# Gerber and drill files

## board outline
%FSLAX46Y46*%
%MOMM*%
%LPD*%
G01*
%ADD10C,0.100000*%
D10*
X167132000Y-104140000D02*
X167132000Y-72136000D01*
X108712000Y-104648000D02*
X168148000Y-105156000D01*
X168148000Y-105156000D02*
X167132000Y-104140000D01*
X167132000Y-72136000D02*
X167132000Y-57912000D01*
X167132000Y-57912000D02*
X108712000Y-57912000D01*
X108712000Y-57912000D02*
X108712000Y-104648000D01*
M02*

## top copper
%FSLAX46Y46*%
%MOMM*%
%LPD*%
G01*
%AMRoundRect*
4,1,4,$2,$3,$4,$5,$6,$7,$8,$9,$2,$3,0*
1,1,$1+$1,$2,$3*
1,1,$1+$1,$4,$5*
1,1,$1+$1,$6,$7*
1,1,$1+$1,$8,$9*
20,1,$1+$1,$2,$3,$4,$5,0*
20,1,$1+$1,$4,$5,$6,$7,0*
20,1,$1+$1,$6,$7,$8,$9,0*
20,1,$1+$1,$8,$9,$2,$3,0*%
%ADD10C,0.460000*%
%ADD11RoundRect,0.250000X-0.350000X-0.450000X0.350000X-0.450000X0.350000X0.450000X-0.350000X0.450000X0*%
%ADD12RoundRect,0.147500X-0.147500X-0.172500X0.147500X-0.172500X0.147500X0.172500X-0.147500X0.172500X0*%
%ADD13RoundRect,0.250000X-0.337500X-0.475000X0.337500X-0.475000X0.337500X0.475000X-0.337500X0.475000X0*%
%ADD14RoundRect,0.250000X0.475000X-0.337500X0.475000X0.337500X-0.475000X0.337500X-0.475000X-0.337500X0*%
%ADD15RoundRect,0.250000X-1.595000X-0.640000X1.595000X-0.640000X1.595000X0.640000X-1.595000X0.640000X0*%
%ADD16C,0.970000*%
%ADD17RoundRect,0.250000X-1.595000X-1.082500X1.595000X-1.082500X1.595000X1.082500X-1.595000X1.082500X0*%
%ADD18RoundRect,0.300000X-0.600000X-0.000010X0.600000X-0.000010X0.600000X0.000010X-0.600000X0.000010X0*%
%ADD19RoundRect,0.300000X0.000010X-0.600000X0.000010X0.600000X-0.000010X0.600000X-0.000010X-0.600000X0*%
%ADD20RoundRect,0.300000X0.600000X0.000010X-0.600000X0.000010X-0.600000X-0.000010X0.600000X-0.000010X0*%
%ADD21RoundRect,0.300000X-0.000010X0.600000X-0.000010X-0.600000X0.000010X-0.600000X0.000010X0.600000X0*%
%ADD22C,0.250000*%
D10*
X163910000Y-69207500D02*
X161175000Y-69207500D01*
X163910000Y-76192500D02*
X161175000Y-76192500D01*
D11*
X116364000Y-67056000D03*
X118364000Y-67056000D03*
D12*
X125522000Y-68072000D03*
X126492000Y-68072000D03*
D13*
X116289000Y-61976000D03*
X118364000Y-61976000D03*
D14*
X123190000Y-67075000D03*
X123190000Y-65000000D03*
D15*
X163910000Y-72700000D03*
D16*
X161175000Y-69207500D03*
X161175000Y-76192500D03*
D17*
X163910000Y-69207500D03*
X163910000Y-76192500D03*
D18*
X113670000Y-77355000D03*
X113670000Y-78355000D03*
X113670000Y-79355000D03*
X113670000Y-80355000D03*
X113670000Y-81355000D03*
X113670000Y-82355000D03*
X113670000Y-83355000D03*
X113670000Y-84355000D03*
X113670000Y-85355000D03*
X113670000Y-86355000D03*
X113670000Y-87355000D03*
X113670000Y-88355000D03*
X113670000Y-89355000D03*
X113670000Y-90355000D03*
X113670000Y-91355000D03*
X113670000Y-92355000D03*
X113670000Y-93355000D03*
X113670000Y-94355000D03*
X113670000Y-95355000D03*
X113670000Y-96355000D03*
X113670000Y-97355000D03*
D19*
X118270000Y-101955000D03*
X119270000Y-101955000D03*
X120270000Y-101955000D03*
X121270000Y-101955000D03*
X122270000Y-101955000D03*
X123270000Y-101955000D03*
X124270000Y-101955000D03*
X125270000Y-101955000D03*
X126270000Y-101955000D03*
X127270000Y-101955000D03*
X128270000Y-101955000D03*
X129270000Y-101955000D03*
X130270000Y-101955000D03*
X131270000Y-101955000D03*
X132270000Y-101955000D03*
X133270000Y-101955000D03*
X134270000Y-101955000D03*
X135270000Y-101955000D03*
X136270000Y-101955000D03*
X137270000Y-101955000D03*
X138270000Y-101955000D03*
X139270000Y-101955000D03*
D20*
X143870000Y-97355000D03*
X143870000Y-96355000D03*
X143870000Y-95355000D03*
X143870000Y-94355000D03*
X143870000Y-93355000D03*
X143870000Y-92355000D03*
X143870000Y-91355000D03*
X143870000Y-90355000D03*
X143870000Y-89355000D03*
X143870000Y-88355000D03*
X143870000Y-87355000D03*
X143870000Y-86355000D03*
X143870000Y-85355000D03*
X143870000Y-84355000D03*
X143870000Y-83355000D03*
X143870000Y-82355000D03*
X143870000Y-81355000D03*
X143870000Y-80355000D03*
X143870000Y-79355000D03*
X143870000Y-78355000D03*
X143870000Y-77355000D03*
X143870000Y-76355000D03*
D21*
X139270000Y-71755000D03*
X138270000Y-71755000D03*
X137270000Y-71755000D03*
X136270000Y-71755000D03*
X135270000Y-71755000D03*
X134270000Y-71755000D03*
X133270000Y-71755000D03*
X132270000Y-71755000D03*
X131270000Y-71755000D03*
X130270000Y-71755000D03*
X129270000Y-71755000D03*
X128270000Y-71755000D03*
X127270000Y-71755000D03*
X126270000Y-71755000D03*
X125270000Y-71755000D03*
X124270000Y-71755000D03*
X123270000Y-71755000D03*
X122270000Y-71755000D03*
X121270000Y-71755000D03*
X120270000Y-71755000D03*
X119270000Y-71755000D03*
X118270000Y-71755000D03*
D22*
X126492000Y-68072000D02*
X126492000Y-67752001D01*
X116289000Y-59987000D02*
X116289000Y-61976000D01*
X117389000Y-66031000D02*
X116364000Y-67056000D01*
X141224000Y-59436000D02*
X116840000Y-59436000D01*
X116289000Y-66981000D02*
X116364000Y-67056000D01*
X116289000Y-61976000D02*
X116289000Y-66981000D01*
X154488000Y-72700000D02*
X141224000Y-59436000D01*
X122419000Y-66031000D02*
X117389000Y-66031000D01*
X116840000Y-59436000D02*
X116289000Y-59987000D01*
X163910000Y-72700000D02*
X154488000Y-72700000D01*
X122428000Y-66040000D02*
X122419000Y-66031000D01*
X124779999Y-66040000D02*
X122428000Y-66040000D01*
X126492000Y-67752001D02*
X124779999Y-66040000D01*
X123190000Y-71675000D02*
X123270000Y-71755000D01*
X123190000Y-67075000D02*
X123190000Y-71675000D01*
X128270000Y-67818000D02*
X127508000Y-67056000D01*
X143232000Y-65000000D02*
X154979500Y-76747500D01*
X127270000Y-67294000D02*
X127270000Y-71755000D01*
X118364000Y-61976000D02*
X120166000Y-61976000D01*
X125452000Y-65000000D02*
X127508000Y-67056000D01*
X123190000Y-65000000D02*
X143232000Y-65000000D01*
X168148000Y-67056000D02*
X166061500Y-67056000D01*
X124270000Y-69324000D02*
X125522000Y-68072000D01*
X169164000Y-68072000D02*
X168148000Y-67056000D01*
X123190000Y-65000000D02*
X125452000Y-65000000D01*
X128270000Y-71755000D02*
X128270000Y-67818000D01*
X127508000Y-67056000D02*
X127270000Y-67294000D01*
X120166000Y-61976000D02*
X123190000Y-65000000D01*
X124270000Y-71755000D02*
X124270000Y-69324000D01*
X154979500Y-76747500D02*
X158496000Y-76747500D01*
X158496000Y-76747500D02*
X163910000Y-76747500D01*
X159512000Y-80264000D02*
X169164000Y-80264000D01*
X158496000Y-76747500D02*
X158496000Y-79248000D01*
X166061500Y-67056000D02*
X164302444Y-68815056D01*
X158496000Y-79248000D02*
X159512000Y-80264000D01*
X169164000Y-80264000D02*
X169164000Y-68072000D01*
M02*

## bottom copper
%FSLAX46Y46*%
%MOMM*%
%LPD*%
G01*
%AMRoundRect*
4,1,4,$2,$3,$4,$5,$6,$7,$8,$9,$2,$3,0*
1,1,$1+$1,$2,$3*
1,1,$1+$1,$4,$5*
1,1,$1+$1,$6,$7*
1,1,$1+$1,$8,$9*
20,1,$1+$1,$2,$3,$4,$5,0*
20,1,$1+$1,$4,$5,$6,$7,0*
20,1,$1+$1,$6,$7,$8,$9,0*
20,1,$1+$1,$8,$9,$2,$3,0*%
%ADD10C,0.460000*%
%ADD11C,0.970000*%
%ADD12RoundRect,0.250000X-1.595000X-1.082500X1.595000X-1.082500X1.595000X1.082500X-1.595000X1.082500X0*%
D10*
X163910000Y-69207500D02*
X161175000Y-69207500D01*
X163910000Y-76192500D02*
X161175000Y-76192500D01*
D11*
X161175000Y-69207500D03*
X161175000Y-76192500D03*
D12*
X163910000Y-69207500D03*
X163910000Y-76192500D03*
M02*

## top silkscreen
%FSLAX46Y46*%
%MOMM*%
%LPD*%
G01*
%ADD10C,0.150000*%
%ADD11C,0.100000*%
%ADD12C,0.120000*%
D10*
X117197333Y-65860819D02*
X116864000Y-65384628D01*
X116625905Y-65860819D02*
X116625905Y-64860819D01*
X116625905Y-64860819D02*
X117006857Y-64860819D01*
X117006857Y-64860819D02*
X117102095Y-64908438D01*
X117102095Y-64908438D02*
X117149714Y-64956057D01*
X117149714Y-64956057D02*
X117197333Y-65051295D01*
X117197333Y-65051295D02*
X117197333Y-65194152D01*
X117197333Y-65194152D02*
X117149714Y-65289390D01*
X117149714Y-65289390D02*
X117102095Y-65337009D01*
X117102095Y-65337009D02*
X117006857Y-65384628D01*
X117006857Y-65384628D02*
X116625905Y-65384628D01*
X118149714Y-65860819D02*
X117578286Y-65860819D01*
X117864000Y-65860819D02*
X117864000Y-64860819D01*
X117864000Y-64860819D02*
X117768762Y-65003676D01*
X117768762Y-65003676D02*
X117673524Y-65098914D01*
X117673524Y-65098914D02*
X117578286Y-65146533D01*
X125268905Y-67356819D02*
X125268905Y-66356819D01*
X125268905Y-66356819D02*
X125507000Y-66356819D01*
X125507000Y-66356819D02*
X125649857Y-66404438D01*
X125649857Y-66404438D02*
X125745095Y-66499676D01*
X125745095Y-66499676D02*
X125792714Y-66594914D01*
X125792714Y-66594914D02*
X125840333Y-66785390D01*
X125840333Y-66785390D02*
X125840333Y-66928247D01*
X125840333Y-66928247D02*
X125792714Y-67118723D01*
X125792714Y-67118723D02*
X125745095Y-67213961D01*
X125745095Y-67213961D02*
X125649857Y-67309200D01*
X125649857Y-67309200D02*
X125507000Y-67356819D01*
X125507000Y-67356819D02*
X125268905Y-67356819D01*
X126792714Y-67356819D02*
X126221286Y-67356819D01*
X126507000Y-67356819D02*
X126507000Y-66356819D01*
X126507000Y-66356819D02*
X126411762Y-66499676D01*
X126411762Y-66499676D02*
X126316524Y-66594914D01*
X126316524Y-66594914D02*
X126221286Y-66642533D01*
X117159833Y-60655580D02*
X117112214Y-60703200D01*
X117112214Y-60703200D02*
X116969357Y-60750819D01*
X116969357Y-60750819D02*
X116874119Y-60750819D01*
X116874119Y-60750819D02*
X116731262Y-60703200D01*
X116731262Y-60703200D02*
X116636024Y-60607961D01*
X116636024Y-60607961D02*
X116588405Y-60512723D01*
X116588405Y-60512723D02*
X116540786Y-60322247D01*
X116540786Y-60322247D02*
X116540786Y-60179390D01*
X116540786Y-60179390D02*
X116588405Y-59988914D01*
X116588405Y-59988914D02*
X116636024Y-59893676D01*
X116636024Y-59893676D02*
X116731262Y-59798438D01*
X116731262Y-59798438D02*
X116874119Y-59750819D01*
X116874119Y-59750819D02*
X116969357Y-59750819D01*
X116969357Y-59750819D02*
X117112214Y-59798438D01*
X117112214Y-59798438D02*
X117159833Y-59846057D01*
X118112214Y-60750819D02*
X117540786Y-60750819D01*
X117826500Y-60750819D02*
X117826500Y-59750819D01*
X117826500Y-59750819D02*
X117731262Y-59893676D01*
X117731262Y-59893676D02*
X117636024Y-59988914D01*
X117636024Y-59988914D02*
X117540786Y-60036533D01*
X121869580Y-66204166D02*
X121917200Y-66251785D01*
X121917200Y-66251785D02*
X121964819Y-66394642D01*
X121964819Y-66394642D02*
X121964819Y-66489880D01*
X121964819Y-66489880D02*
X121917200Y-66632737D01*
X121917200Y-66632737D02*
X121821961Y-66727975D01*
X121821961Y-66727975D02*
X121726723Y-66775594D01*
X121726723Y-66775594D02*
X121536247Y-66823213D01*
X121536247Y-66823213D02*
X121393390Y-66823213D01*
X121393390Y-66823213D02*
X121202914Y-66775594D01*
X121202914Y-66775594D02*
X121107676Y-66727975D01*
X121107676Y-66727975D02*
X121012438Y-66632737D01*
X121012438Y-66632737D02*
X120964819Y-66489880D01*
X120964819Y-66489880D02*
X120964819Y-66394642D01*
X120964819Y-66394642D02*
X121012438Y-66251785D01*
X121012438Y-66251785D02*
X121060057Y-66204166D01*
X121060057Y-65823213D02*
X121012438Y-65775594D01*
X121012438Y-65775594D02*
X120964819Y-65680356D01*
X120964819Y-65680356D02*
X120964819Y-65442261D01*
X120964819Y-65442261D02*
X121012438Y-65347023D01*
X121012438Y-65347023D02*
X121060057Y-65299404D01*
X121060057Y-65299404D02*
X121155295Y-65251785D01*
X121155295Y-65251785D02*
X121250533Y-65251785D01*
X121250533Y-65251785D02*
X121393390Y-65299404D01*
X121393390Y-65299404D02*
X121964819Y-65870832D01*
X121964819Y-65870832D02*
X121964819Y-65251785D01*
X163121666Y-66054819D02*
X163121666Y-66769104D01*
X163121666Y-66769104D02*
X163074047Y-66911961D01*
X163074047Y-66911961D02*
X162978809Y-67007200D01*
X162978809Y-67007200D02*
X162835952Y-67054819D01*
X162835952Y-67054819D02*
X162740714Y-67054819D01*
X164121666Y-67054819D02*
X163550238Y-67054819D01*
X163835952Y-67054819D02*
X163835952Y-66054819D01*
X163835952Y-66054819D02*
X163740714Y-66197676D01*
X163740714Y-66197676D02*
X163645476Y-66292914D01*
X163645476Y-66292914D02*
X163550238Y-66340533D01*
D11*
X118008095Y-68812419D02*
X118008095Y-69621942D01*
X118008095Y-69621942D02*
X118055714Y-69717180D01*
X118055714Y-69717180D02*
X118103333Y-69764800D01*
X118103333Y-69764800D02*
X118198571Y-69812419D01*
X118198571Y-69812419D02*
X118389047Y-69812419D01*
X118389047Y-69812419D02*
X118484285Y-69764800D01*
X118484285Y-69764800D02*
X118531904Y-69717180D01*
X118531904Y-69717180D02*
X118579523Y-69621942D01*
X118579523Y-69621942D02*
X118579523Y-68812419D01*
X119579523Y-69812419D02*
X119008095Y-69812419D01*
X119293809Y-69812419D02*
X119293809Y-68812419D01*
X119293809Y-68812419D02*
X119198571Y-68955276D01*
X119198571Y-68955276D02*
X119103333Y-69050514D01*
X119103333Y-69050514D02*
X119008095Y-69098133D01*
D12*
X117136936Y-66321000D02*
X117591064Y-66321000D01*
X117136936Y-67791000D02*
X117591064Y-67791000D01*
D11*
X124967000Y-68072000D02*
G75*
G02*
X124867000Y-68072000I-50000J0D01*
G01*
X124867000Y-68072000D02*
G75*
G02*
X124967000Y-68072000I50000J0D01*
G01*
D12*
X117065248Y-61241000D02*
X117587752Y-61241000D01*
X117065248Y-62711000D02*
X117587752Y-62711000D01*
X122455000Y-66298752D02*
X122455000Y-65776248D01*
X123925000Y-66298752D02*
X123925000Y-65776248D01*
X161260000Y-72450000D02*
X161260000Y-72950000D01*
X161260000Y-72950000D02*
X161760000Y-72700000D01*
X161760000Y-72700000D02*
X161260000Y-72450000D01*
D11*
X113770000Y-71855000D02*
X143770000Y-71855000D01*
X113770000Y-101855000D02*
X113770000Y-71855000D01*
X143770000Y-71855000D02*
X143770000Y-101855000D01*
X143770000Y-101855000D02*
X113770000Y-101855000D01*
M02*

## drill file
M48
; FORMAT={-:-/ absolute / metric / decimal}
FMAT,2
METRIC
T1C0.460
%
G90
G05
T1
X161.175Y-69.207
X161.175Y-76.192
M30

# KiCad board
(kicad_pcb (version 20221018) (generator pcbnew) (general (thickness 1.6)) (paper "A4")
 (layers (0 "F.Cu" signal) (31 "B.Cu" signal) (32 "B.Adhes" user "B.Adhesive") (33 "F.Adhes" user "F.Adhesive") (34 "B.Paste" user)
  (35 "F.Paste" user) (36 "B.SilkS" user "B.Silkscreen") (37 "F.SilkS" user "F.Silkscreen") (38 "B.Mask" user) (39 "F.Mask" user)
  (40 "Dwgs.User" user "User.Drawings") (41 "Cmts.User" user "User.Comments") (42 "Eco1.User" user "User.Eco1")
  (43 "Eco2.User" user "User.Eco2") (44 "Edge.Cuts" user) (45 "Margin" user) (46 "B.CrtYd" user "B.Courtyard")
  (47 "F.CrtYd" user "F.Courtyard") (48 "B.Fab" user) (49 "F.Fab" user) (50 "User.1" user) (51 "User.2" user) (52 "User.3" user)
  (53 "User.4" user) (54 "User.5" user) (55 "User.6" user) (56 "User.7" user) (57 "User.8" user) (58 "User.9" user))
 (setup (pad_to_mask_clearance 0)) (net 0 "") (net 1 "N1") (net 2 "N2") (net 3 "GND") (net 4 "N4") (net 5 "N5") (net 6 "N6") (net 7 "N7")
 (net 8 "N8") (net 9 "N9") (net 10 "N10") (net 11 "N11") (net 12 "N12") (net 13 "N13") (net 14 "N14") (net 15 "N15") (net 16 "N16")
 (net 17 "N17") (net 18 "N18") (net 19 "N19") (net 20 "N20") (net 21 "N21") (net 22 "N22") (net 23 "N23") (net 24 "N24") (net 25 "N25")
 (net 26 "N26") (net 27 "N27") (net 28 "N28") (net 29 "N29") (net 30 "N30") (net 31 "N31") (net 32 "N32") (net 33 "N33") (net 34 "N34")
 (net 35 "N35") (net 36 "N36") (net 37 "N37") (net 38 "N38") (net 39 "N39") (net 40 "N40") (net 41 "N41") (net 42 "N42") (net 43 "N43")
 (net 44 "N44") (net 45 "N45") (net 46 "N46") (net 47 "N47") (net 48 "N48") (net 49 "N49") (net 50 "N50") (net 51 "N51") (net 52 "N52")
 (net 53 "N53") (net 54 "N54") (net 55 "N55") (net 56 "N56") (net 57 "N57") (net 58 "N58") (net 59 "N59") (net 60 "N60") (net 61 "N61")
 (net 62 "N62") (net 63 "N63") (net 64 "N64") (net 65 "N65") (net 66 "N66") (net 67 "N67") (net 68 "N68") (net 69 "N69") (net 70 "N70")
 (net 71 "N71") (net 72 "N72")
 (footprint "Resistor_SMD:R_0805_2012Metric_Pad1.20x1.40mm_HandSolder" (layer "F.Cu") (at 117.364 67.056)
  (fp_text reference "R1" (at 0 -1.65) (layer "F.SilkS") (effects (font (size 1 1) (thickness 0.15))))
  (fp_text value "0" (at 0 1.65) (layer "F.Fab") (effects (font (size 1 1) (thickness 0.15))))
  (fp_line (start -0.227064 -0.735) (end 0.227064 -0.735) (stroke (width 0.12) (type solid)) (layer "F.SilkS"))
  (fp_line (start -0.227064 0.735) (end 0.227064 0.735) (stroke (width 0.12) (type solid)) (layer "F.SilkS"))
  (pad "1" smd roundrect (at -1 0) (size 1.2 1.4) (layers "F.Cu" "F.Paste" "F.Mask") (roundrect_rratio 0.208333) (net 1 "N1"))
  (pad "2" smd roundrect (at 1 0) (size 1.2 1.4) (layers "F.Cu" "F.Paste" "F.Mask") (roundrect_rratio 0.208333) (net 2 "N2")))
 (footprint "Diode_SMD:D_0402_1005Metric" (layer "F.Cu") (at 126.007 68.072)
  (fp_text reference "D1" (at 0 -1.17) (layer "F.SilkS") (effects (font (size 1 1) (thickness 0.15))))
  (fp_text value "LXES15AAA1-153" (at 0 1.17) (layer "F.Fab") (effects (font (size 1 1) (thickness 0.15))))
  (fp_circle (center -1.09 0) (end -1.04 0) (stroke (width 0.1) (type solid)) (fill none) (layer "F.SilkS"))
  (pad "1" smd roundrect (at -0.485 0) (size 0.59 0.64) (layers "F.Cu" "F.Paste" "F.Mask") (roundrect_rratio 0.25) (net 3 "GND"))
  (pad "2" smd roundrect (at 0.485 0) (size 0.59 0.64) (layers "F.Cu" "F.Paste" "F.Mask") (roundrect_rratio 0.25) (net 1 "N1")))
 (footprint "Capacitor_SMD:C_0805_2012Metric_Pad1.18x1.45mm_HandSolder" (layer "F.Cu") (at 117.3265 61.976)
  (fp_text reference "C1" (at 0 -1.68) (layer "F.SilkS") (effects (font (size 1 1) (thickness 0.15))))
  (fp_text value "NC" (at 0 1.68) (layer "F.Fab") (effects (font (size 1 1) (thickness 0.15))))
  (fp_line (start -0.261252 -0.735) (end 0.261252 -0.735) (stroke (width 0.12) (type solid)) (layer "F.SilkS"))
  (fp_line (start -0.261252 0.735) (end 0.261252 0.735) (stroke (width 0.12) (type solid)) (layer "F.SilkS"))
  (pad "1" smd roundrect (at -1.0375 0) (size 1.175 1.45) (layers "F.Cu" "F.Paste" "F.Mask") (roundrect_rratio 0.212766) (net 1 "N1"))
  (pad "2" smd roundrect (at 1.0375 0) (size 1.175 1.45) (layers "F.Cu" "F.Paste" "F.Mask") (roundrect_rratio 0.212766) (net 3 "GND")))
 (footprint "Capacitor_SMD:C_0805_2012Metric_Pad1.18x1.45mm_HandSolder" (layer "F.Cu") (at 123.19 66.0375 90)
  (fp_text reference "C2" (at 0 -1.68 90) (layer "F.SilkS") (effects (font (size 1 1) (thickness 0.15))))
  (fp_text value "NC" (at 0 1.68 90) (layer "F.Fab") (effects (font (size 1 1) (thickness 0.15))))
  (fp_line (start -0.261252 -0.735) (end 0.261252 -0.735) (stroke (width 0.12) (type solid)) (layer "F.SilkS"))
  (fp_line (start -0.261252 0.735) (end 0.261252 0.735) (stroke (width 0.12) (type solid)) (layer "F.SilkS"))
  (pad "1" smd roundrect (at -1.0375 0 90) (size 1.175 1.45) (layers "F.Cu" "F.Paste" "F.Mask") (roundrect_rratio 0.212766) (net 2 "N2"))
  (pad "2" smd roundrect (at 1.0375 0 90) (size 1.175 1.45) (layers "F.Cu" "F.Paste" "F.Mask") (roundrect_rratio 0.212766) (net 3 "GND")))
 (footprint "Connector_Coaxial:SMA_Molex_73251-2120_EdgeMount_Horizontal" (layer "F.Cu") (at 164.16 72.7)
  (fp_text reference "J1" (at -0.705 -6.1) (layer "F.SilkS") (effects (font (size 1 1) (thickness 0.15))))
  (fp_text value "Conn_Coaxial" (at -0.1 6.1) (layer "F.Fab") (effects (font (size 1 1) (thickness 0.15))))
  (fp_line (start -0.25 -3.4925) (end -2.985 -3.4925) (stroke (width 0.46) (type default)) (layer "F.Cu"))
  (fp_line (start -0.25 3.4925) (end -2.985 3.4925) (stroke (width 0.46) (type default)) (layer "F.Cu"))
  (fp_line (start -0.25 -3.4925) (end -2.985 -3.4925) (stroke (width 0.46) (type default)) (layer "B.Cu"))
  (fp_line (start -0.25 3.4925) (end -2.985 3.4925) (stroke (width 0.46) (type default)) (layer "B.Cu"))
  (fp_line (start -2.9 -0.25) (end -2.9 0.25) (stroke (width 0.12) (type solid)) (layer "F.SilkS"))
  (fp_line (start -2.9 0.25) (end -2.4 0) (stroke (width 0.12) (type solid)) (layer "F.SilkS"))
  (fp_line (start -2.4 0) (end -2.9 -0.25) (stroke (width 0.12) (type solid)) (layer "F.SilkS"))
  (pad "1" smd roundrect (at -0.25 0) (size 3.69 1.78) (layers "F.Cu" "F.Paste" "F.Mask") (roundrect_rratio 0.1404494382) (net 1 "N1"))
  (pad "2" thru_hole circle (at -2.985 -3.4925) (size 0.97 0.97) (drill 0.46) (layers "*.Cu") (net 3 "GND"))
  (pad "2" thru_hole circle (at -2.985 3.4925) (size 0.97 0.97) (drill 0.46) (layers "*.Cu") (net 3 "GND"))
  (pad "2" smd roundrect (at -0.25 -3.4925) (size 3.69 2.665) (layers "F.Cu" "F.Paste" "F.Mask") (roundrect_rratio 0.09380863039)
   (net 3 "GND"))
  (pad "2" smd roundrect (at -0.25 -3.4925) (size 3.69 2.665) (layers "B.Cu" "B.Paste" "B.Mask") (roundrect_rratio 0.09380863039)
   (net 3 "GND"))
  (pad "2" smd roundrect (at -0.25 3.4925) (size 3.69 2.665) (layers "F.Cu" "F.Paste" "F.Mask") (roundrect_rratio 0.09380863039)
   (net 3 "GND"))
  (pad "2" smd roundrect (at -0.25 3.4925) (size 3.69 2.665) (layers "B.Cu" "B.Paste" "B.Mask") (roundrect_rratio 0.09380863039)
   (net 3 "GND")))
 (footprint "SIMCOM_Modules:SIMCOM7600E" (layer "F.Cu") (at 128.77 86.855)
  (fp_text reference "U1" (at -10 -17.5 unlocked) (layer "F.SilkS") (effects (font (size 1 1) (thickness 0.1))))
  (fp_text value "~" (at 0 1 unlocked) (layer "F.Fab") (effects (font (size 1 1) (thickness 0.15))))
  (fp_line (start -15 -15) (end 15 -15) (stroke (width 0.1) (type default)) (layer "F.SilkS"))
  (fp_line (start -15 15) (end -15 -15) (stroke (width 0.1) (type default)) (layer "F.SilkS"))
  (fp_line (start 15 -15) (end 15 15) (stroke (width 0.1) (type default)) (layer "F.SilkS"))
  (fp_line (start 15 15) (end -15 15) (stroke (width 0.1) (type default)) (layer "F.SilkS"))
  (pad "1" smd roundrect (at -15.1 -9.5) (size 1.8 0.6) (layers "F.Cu" "F.Paste" "F.Mask") (roundrect_rratio 0.5) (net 3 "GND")
   (thermal_bridge_angle 45))
  (pad "2" smd roundrect (at -15.1 -8.5) (size 1.8 0.6) (layers "F.Cu" "F.Paste" "F.Mask") (roundrect_rratio 0.5) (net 3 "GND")
   (thermal_bridge_angle 45))
  (pad "3" smd roundrect (at -15.1 -7.5) (size 1.8 0.6) (layers "F.Cu" "F.Paste" "F.Mask") (roundrect_rratio 0.5) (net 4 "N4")
   (thermal_bridge_angle 45))
  (pad "4" smd roundrect (at -15.1 -6.5) (size 1.8 0.6) (layers "F.Cu" "F.Paste" "F.Mask") (roundrect_rratio 0.5) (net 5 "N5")
   (thermal_bridge_angle 45))
  (pad "5" smd roundrect (at -15.1 -5.5) (size 1.8 0.6) (layers "F.Cu" "F.Paste" "F.Mask") (roundrect_rratio 0.5) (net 3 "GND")
   (thermal_bridge_angle 45))
  (pad "6" smd roundrect (at -15.1 -4.5) (size 1.8 0.6) (layers "F.Cu" "F.Paste" "F.Mask") (roundrect_rratio 0.5) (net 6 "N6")
   (thermal_bridge_angle 45))
  (pad "7" smd roundrect (at -15.1 -3.5) (size 1.8 0.6) (layers "F.Cu" "F.Paste" "F.Mask") (roundrect_rratio 0.5) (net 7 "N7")
   (thermal_bridge_angle 45))
  (pad "8" smd roundrect (at -15.1 -2.5) (size 1.8 0.6) (layers "F.Cu" "F.Paste" "F.Mask") (roundrect_rratio 0.5) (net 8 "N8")
   (thermal_bridge_angle 45))
  (pad "9" smd roundrect (at -15.1 -1.5) (size 1.8 0.6) (layers "F.Cu" "F.Paste" "F.Mask") (roundrect_rratio 0.5) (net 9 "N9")
   (thermal_bridge_angle 45))
  (pad "10" smd roundrect (at -15.1 -0.5) (size 1.8 0.6) (layers "F.Cu" "F.Paste" "F.Mask") (roundrect_rratio 0.5) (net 3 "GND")
   (thermal_bridge_angle 45))
  (pad "11" smd roundrect (at -15.1 0.5) (size 1.8 0.6) (layers "F.Cu" "F.Paste" "F.Mask") (roundrect_rratio 0.5) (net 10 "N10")
   (thermal_bridge_angle 45))
  (pad "12" smd roundrect (at -15.1 1.5) (size 1.8 0.6) (layers "F.Cu" "F.Paste" "F.Mask") (roundrect_rratio 0.5) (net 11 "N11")
   (thermal_bridge_angle 45))
  (pad "13" smd roundrect (at -15.1 2.5) (size 1.8 0.6) (layers "F.Cu" "F.Paste" "F.Mask") (roundrect_rratio 0.5) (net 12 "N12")
   (thermal_bridge_angle 45))
  (pad "14" smd roundrect (at -15.1 3.5) (size 1.8 0.6) (layers "F.Cu" "F.Paste" "F.Mask") (roundrect_rratio 0.5) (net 3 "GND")
   (thermal_bridge_angle 45))
  (pad "15" smd roundrect (at -15.1 4.5) (size 1.8 0.6) (layers "F.Cu" "F.Paste" "F.Mask") (roundrect_rratio 0.5) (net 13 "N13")
   (thermal_bridge_angle 45))
  (pad "16" smd roundrect (at -15.1 5.5) (size 1.8 0.6) (layers "F.Cu" "F.Paste" "F.Mask") (roundrect_rratio 0.5) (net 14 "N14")
   (thermal_bridge_angle 45))
  (pad "17" smd roundrect (at -15.1 6.5) (size 1.8 0.6) (layers "F.Cu" "F.Paste" "F.Mask") (roundrect_rratio 0.5) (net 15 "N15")
   (thermal_bridge_angle 45))
  (pad "18" smd roundrect (at -15.1 7.5) (size 1.8 0.6) (layers "F.Cu" "F.Paste" "F.Mask") (roundrect_rratio 0.5) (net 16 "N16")
   (thermal_bridge_angle 45))
  (pad "19" smd roundrect (at -15.1 8.5) (size 1.8 0.6) (layers "F.Cu" "F.Paste" "F.Mask") (roundrect_rratio 0.5) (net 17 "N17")
   (thermal_bridge_angle 45))
  (pad "20" smd roundrect (at -15.1 9.5) (size 1.8 0.6) (layers "F.Cu" "F.Paste" "F.Mask") (roundrect_rratio 0.5) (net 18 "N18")
   (thermal_bridge_angle 45))
  (pad "21" smd roundrect (at -15.1 10.5) (size 1.8 0.6) (layers "F.Cu" "F.Paste" "F.Mask") (roundrect_rratio 0.5) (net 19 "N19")
   (thermal_bridge_angle 45))
  (pad "22" smd roundrect (at -10.5 15.1 90) (size 1.8 0.6) (layers "F.Cu" "F.Paste" "F.Mask") (roundrect_rratio 0.5) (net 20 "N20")
   (thermal_bridge_angle 45))
  (pad "23" smd roundrect (at -9.5 15.1 90) (size 1.8 0.6) (layers "F.Cu" "F.Paste" "F.Mask") (roundrect_rratio 0.5) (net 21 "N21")
   (thermal_bridge_angle 45))
  (pad "24" smd roundrect (at -8.5 15.1 90) (size 1.8 0.6) (layers "F.Cu" "F.Paste" "F.Mask") (roundrect_rratio 0.5) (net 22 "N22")
   (thermal_bridge_angle 45))
  (pad "25" smd roundrect (at -7.5 15.1 90) (size 1.8 0.6) (layers "F.Cu" "F.Paste" "F.Mask") (roundrect_rratio 0.5) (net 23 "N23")
   (thermal_bridge_angle 45))
  (pad "26" smd roundrect (at -6.5 15.1 90) (size 1.8 0.6) (layers "F.Cu" "F.Paste" "F.Mask") (roundrect_rratio 0.5) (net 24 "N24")
   (thermal_bridge_angle 45))
  (pad "27" smd roundrect (at -5.5 15.1 90) (size 1.8 0.6) (layers "F.Cu" "F.Paste" "F.Mask") (roundrect_rratio 0.5) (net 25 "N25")
   (thermal_bridge_angle 45))
  (pad "28" smd roundrect (at -4.5 15.1 90) (size 1.8 0.6) (layers "F.Cu" "F.Paste" "F.Mask") (roundrect_rratio 0.5) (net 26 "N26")
   (thermal_bridge_angle 45))
  (pad "29" smd roundrect (at -3.5 15.1 90) (size 1.8 0.6) (layers "F.Cu" "F.Paste" "F.Mask") (roundrect_rratio 0.5) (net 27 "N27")
   (thermal_bridge_angle 45))
  (pad "30" smd roundrect (at -2.5 15.1 90) (size 1.8 0.6) (layers "F.Cu" "F.Paste" "F.Mask") (roundrect_rratio 0.5) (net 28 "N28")
   (thermal_bridge_angle 45))
  (pad "31" smd roundrect (at -1.5 15.1 90) (size 1.8 0.6) (layers "F.Cu" "F.Paste" "F.Mask") (roundrect_rratio 0.5) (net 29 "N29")
   (thermal_bridge_angle 45))
  (pad "32" smd roundrect (at -0.5 15.1 90) (size 1.8 0.6) (layers "F.Cu" "F.Paste" "F.Mask") (roundrect_rratio 0.5) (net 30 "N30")
   (thermal_bridge_angle 45))
  (pad "33" smd roundrect (at 0.5 15.1 90) (size 1.8 0.6) (layers "F.Cu" "F.Paste" "F.Mask") (roundrect_rratio 0.5) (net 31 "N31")
   (thermal_bridge_angle 45))
  (pad "34" smd roundrect (at 1.5 15.1 90) (size 1.8 0.6) (layers "F.Cu" "F.Paste" "F.Mask") (roundrect_rratio 0.5) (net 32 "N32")
   (thermal_bridge_angle 45))
  (pad "35" smd roundrect (at 2.5 15.1 90) (size 1.8 0.6) (layers "F.Cu" "F.Paste" "F.Mask") (roundrect_rratio 0.5) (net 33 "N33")
   (thermal_bridge_angle 45))
  (pad "36" smd roundrect (at 3.5 15.1 90) (size 1.8 0.6) (layers "F.Cu" "F.Paste" "F.Mask") (roundrect_rratio 0.5) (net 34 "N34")
   (thermal_bridge_angle 45))
  (pad "37" smd roundrect (at 4.5 15.1 90) (size 1.8 0.6) (layers "F.Cu" "F.Paste" "F.Mask") (roundrect_rratio 0.5) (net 3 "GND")
   (thermal_bridge_angle 45))
  (pad "38" smd roundrect (at 5.5 15.1 90) (size 1.8 0.6) (layers "F.Cu" "F.Paste" "F.Mask") (roundrect_rratio 0.5) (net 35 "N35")
   (thermal_bridge_angle 45))
  (pad "39" smd roundrect (at 6.5 15.1 90) (size 1.8 0.6) (layers "F.Cu" "F.Paste" "F.Mask") (roundrect_rratio 0.5) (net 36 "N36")
   (thermal_bridge_angle 45))
  (pad "40" smd roundrect (at 7.5 15.1 90) (size 1.8 0.6) (layers "F.Cu" "F.Paste" "F.Mask") (roundrect_rratio 0.5) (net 3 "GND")
   (thermal_bridge_angle 45))
  (pad "41" smd roundrect (at 8.5 15.1 90) (size 1.8 0.6) (layers "F.Cu" "F.Paste" "F.Mask") (roundrect_rratio 0.5) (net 3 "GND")
   (thermal_bridge_angle 45))
  (pad "42" smd roundrect (at 9.5 15.1 90) (size 1.8 0.6) (layers "F.Cu" "F.Paste" "F.Mask") (roundrect_rratio 0.5) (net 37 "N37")
   (thermal_bridge_angle 45))
  (pad "43" smd roundrect (at 10.5 15.1 90) (size 1.8 0.6) (layers "F.Cu" "F.Paste" "F.Mask") (roundrect_rratio 0.5) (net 3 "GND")
   (thermal_bridge_angle 45))
  (pad "44" smd roundrect (at 15.1 10.5 180) (size 1.8 0.6) (layers "F.Cu" "F.Paste" "F.Mask") (roundrect_rratio 0.5) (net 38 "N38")
   (thermal_bridge_angle 45))
  (pad "45" smd roundrect (at 15.1 9.5 180) (size 1.8 0.6) (layers "F.Cu" "F.Paste" "F.Mask") (roundrect_rratio 0.5) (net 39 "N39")
   (thermal_bridge_angle 45))
  (pad "46" smd roundrect (at 15.1 8.5 180) (size 1.8 0.6) (layers "F.Cu" "F.Paste" "F.Mask") (roundrect_rratio 0.5) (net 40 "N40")
   (thermal_bridge_angle 45))
  (pad "47" smd roundrect (at 15.1 7.5 180) (size 1.8 0.6) (layers "F.Cu" "F.Paste" "F.Mask") (roundrect_rratio 0.5) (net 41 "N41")
   (thermal_bridge_angle 45))
  (pad "48" smd roundrect (at 15.1 6.5 180) (size 1.8 0.6) (layers "F.Cu" "F.Paste" "F.Mask") (roundrect_rratio 0.5) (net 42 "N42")
   (thermal_bridge_angle 45))
  (pad "49" smd roundrect (at 15.1 5.5 180) (size 1.8 0.6) (layers "F.Cu" "F.Paste" "F.Mask") (roundrect_rratio 0.5) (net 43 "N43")
   (thermal_bridge_angle 45))
  (pad "50" smd roundrect (at 15.1 4.5 180) (size 1.8 0.6) (layers "F.Cu" "F.Paste" "F.Mask") (roundrect_rratio 0.5) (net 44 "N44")
   (thermal_bridge_angle 45))
  (pad "51" smd roundrect (at 15.1 3.5 180) (size 1.8 0.6) (layers "F.Cu" "F.Paste" "F.Mask") (roundrect_rratio 0.5) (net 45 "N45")
   (thermal_bridge_angle 45))
  (pad "52" smd roundrect (at 15.1 2.5 180) (size 1.8 0.6) (layers "F.Cu" "F.Paste" "F.Mask") (roundrect_rratio 0.5) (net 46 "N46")
   (thermal_bridge_angle 45))
  (pad "53" smd roundrect (at 15.1 1.5 180) (size 1.8 0.6) (layers "F.Cu" "F.Paste" "F.Mask") (roundrect_rratio 0.5) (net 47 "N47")
   (thermal_bridge_angle 45))
  (pad "54" smd roundrect (at 15.1 0.5 180) (size 1.8 0.6) (layers "F.Cu" "F.Paste" "F.Mask") (roundrect_rratio 0.5) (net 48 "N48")
   (thermal_bridge_angle 45))
  (pad "55" smd roundrect (at 15.1 -0.5 180) (size 1.8 0.6) (layers "F.Cu" "F.Paste" "F.Mask") (roundrect_rratio 0.5) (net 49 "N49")
   (thermal_bridge_angle 45))
  (pad "56" smd roundrect (at 15.1 -1.5 180) (size 1.8 0.6) (layers "F.Cu" "F.Paste" "F.Mask") (roundrect_rratio 0.5) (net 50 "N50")
   (thermal_bridge_angle 45))
  (pad "57" smd roundrect (at 15.1 -2.5 180) (size 1.8 0.6) (layers "F.Cu" "F.Paste" "F.Mask") (roundrect_rratio 0.5) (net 3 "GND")
   (thermal_bridge_angle 45))
  (pad "58" smd roundrect (at 15.1 -3.5 180) (size 1.8 0.6) (layers "F.Cu" "F.Paste" "F.Mask") (roundrect_rratio 0.5) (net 3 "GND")
   (thermal_bridge_angle 45))
  (pad "59" smd roundrect (at 15.1 -4.5 180) (size 1.8 0.6) (layers "F.Cu" "F.Paste" "F.Mask") (roundrect_rratio 0.5) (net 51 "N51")
   (thermal_bridge_angle 45))
  (pad "60" smd roundrect (at 15.1 -5.5 180) (size 1.8 0.6) (layers "F.Cu" "F.Paste" "F.Mask") (roundrect_rratio 0.5) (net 3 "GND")
   (thermal_bridge_angle 45))
  (pad "61" smd roundrect (at 15.1 -6.5 180) (size 1.8 0.6) (layers "F.Cu" "F.Paste" "F.Mask") (roundrect_rratio 0.5) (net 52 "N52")
   (thermal_bridge_angle 45))
  (pad "62" smd roundrect (at 15.1 -7.5 180) (size 1.8 0.6) (layers "F.Cu" "F.Paste" "F.Mask") (roundrect_rratio 0.5) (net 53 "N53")
   (thermal_bridge_angle 45))
  (pad "63" smd roundrect (at 15.1 -8.5 180) (size 1.8 0.6) (layers "F.Cu" "F.Paste" "F.Mask") (roundrect_rratio 0.5) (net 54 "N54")
   (thermal_bridge_angle 45))
  (pad "64" smd roundrect (at 15.1 -9.5 180) (size 1.8 0.6) (layers "F.Cu" "F.Paste" "F.Mask") (roundrect_rratio 0.5) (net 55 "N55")
   (thermal_bridge_angle 45))
  (pad "65" smd roundrect (at 15.1 -10.5 180) (size 1.8 0.6) (layers "F.Cu" "F.Paste" "F.Mask") (roundrect_rratio 0.5) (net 3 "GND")
   (thermal_bridge_angle 45))
  (pad "66" smd roundrect (at 10.5 -15.1 270) (size 1.8 0.6) (layers "F.Cu" "F.Paste" "F.Mask") (roundrect_rratio 0.5) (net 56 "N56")
   (thermal_bridge_angle 45))
  (pad "67" smd roundrect (at 9.5 -15.1 270) (size 1.8 0.6) (layers "F.Cu" "F.Paste" "F.Mask") (roundrect_rratio 0.5) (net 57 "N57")
   (thermal_bridge_angle 45))
  (pad "68" smd roundrect (at 8.5 -15.1 270) (size 1.8 0.6) (layers "F.Cu" "F.Paste" "F.Mask") (roundrect_rratio 0.5) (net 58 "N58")
   (thermal_bridge_angle 45))
  (pad "69" smd roundrect (at 7.5 -15.1 270) (size 1.8 0.6) (layers "F.Cu" "F.Paste" "F.Mask") (roundrect_rratio 0.5) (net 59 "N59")
   (thermal_bridge_angle 45))
  (pad "70" smd roundrect (at 6.5 -15.1 270) (size 1.8 0.6) (layers "F.Cu" "F.Paste" "F.Mask") (roundrect_rratio 0.5) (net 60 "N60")
   (thermal_bridge_angle 45))
  (pad "71" smd roundrect (at 5.5 -15.1 270) (size 1.8 0.6) (layers "F.Cu" "F.Paste" "F.Mask") (roundrect_rratio 0.5) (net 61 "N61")
   (thermal_bridge_angle 45))
  (pad "72" smd roundrect (at 4.5 -15.1 270) (size 1.8 0.6) (layers "F.Cu" "F.Paste" "F.Mask") (roundrect_rratio 0.5) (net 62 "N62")
   (thermal_bridge_angle 45))
  (pad "73" smd roundrect (at 3.5 -15.1 270) (size 1.8 0.6) (layers "F.Cu" "F.Paste" "F.Mask") (roundrect_rratio 0.5) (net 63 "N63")
   (thermal_bridge_angle 45))
  (pad "74" smd roundrect (at 2.5 -15.1 270) (size 1.8 0.6) (layers "F.Cu" "F.Paste" "F.Mask") (roundrect_rratio 0.5) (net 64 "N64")
   (thermal_bridge_angle 45))
  (pad "75" smd roundrect (at 1.5 -15.1 270) (size 1.8 0.6) (layers "F.Cu" "F.Paste" "F.Mask") (roundrect_rratio 0.5) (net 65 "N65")
   (thermal_bridge_angle 45))
  (pad "76" smd roundrect (at 0.5 -15.1 270) (size 1.8 0.6) (layers "F.Cu" "F.Paste" "F.Mask") (roundrect_rratio 0.5) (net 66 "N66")
   (thermal_bridge_angle 45))
  (pad "77" smd roundrect (at -0.5 -15.1 270) (size 1.8 0.6) (layers "F.Cu" "F.Paste" "F.Mask") (roundrect_rratio 0.5) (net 3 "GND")
   (thermal_bridge_angle 45))
  (pad "78" smd roundrect (at -1.5 -15.1 270) (size 1.8 0.6) (layers "F.Cu" "F.Paste" "F.Mask") (roundrect_rratio 0.5) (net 3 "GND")
   (thermal_bridge_angle 45))
  (pad "79" smd roundrect (at -2.5 -15.1 270) (size 1.8 0.6) (layers "F.Cu" "F.Paste" "F.Mask") (roundrect_rratio 0.5) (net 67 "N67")
   (thermal_bridge_angle 45))
  (pad "80" smd roundrect (at -3.5 -15.1 270) (size 1.8 0.6) (layers "F.Cu" "F.Paste" "F.Mask") (roundrect_rratio 0.5) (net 3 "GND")
   (thermal_bridge_angle 45))
  (pad "81" smd roundrect (at -4.5 -15.1 270) (size 1.8 0.6) (layers "F.Cu" "F.Paste" "F.Mask") (roundrect_rratio 0.5) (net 3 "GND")
   (thermal_bridge_angle 45))
  (pad "82" smd roundrect (at -5.5 -15.1 270) (size 1.8 0.6) (layers "F.Cu" "F.Paste" "F.Mask") (roundrect_rratio 0.5) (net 2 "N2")
   (thermal_bridge_angle 45))
  (pad "83" smd roundrect (at -6.5 -15.1 270) (size 1.8 0.6) (layers "F.Cu" "F.Paste" "F.Mask") (roundrect_rratio 0.5) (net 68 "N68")
   (thermal_bridge_angle 45))
  (pad "84" smd roundrect (at -7.5 -15.1 270) (size 1.8 0.6) (layers "F.Cu" "F.Paste" "F.Mask") (roundrect_rratio 0.5) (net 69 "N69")
   (thermal_bridge_angle 45))
  (pad "85" smd roundrect (at -8.5 -15.1 270) (size 1.8 0.6) (layers "F.Cu" "F.Paste" "F.Mask") (roundrect_rratio 0.5) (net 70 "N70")
   (thermal_bridge_angle 45))
  (pad "86" smd roundrect (at -9.5 -15.1 270) (size 1.8 0.6) (layers "F.Cu" "F.Paste" "F.Mask") (roundrect_rratio 0.5) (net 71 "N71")
   (thermal_bridge_angle 45))
  (pad "87" smd roundrect (at -10.5 -15.1 270) (size 1.8 0.6) (layers "F.Cu" "F.Paste" "F.Mask") (roundrect_rratio 0.5) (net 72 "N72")
   (thermal_bridge_angle 45))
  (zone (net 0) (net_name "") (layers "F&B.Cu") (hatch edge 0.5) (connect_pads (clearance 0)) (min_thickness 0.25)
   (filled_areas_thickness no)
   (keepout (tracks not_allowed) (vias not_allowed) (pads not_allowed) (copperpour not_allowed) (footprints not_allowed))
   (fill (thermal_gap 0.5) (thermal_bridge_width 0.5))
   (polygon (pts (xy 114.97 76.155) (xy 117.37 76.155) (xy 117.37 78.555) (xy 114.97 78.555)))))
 (gr_line (start 167.132 104.14) (end 167.132 72.136) (stroke (width 0.1) (type default)) (layer "Edge.Cuts"))
 (gr_line (start 108.712 104.648) (end 168.148 105.156) (stroke (width 0.1) (type default)) (layer "Edge.Cuts"))
 (gr_line (start 168.148 105.156) (end 167.132 104.14) (stroke (width 0.1) (type default)) (layer "Edge.Cuts"))
 (gr_line (start 167.132 72.136) (end 167.132 57.912) (stroke (width 0.1) (type default)) (layer "Edge.Cuts"))
 (gr_line (start 167.132 57.912) (end 108.712 57.912) (stroke (width 0.1) (type default)) (layer "Edge.Cuts"))
 (gr_line (start 108.712 57.912) (end 108.712 104.648) (stroke (width 0.1) (type default)) (layer "Edge.Cuts"))
 (segment (start 126.492 68.072) (end 126.492 67.752001) (width 0.25) (layer "F.Cu") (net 1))
 (segment (start 116.289 59.987) (end 116.289 61.976) (width 0.25) (layer "F.Cu") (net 1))
 (segment (start 117.389 66.031) (end 116.364 67.056) (width 0.25) (layer "F.Cu") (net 1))
 (segment (start 141.224 59.436) (end 116.84 59.436) (width 0.25) (layer "F.Cu") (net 1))
 (segment (start 116.289 66.981) (end 116.364 67.056) (width 0.25) (layer "F.Cu") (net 1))
 (segment (start 116.289 61.976) (end 116.289 66.981) (width 0.25) (layer "F.Cu") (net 1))
 (segment (start 154.488 72.7) (end 141.224 59.436) (width 0.25) (layer "F.Cu") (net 1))
 (segment (start 122.419 66.031) (end 117.389 66.031) (width 0.25) (layer "F.Cu") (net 1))
 (segment (start 116.84 59.436) (end 116.289 59.987) (width 0.25) (layer "F.Cu") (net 1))
 (segment (start 163.91 72.7) (end 154.488 72.7) (width 0.25) (layer "F.Cu") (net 1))
 (segment (start 122.428 66.04) (end 122.419 66.031) (width 0.25) (layer "F.Cu") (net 1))
 (segment (start 124.779999 66.04) (end 122.428 66.04) (width 0.25) (layer "F.Cu") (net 1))
 (segment (start 126.492 67.752001) (end 124.779999 66.04) (width 0.25) (layer "F.Cu") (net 1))
 (segment (start 123.19 71.675) (end 123.27 71.755) (width 0.25) (layer "F.Cu") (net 2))
 (segment (start 123.19 67.075) (end 123.19 71.675) (width 0.25) (layer "F.Cu") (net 2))
 (segment (start 128.27 67.818) (end 127.508 67.056) (width 0.25) (layer "F.Cu") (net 3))
 (segment (start 143.232 65) (end 154.9795 76.7475) (width 0.25) (layer "F.Cu") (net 3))
 (segment (start 127.27 67.294) (end 127.27 71.755) (width 0.25) (layer "F.Cu") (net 3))
 (segment (start 118.364 61.976) (end 120.166 61.976) (width 0.25) (layer "F.Cu") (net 3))
 (segment (start 125.452 65) (end 127.508 67.056) (width 0.25) (layer "F.Cu") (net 3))
 (segment (start 123.19 65) (end 143.232 65) (width 0.25) (layer "F.Cu") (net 3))
 (segment (start 168.148 67.056) (end 166.0615 67.056) (width 0.25) (layer "F.Cu") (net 3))
 (segment (start 124.27 69.324) (end 125.522 68.072) (width 0.25) (layer "F.Cu") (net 3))
 (segment (start 169.164 68.072) (end 168.148 67.056) (width 0.25) (layer "F.Cu") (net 3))
 (segment (start 123.19 65) (end 125.452 65) (width 0.25) (layer "F.Cu") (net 3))
 (segment (start 128.27 71.755) (end 128.27 67.818) (width 0.25) (layer "F.Cu") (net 3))
 (segment (start 127.508 67.056) (end 127.27 67.294) (width 0.25) (layer "F.Cu") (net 3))
 (segment (start 120.166 61.976) (end 123.19 65) (width 0.25) (layer "F.Cu") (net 3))
 (segment (start 124.27 71.755) (end 124.27 69.324) (width 0.25) (layer "F.Cu") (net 3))
 (segment (start 154.9795 76.7475) (end 158.496 76.7475) (width 0.25) (layer "F.Cu") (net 3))
 (segment (start 158.496 76.7475) (end 163.91 76.7475) (width 0.25) (layer "F.Cu") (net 3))
 (segment (start 159.512 80.264) (end 169.164 80.264) (width 0.25) (layer "F.Cu") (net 3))
 (segment (start 158.496 76.7475) (end 158.496 79.248) (width 0.25) (layer "F.Cu") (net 3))
 (segment (start 166.0615 67.056) (end 164.302444 68.815056) (width 0.25) (layer "F.Cu") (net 3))
 (segment (start 158.496 79.248) (end 159.512 80.264) (width 0.25) (layer "F.Cu") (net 3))
 (segment (start 169.164 80.264) (end 169.164 68.072) (width 0.25) (layer "F.Cu") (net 3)))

